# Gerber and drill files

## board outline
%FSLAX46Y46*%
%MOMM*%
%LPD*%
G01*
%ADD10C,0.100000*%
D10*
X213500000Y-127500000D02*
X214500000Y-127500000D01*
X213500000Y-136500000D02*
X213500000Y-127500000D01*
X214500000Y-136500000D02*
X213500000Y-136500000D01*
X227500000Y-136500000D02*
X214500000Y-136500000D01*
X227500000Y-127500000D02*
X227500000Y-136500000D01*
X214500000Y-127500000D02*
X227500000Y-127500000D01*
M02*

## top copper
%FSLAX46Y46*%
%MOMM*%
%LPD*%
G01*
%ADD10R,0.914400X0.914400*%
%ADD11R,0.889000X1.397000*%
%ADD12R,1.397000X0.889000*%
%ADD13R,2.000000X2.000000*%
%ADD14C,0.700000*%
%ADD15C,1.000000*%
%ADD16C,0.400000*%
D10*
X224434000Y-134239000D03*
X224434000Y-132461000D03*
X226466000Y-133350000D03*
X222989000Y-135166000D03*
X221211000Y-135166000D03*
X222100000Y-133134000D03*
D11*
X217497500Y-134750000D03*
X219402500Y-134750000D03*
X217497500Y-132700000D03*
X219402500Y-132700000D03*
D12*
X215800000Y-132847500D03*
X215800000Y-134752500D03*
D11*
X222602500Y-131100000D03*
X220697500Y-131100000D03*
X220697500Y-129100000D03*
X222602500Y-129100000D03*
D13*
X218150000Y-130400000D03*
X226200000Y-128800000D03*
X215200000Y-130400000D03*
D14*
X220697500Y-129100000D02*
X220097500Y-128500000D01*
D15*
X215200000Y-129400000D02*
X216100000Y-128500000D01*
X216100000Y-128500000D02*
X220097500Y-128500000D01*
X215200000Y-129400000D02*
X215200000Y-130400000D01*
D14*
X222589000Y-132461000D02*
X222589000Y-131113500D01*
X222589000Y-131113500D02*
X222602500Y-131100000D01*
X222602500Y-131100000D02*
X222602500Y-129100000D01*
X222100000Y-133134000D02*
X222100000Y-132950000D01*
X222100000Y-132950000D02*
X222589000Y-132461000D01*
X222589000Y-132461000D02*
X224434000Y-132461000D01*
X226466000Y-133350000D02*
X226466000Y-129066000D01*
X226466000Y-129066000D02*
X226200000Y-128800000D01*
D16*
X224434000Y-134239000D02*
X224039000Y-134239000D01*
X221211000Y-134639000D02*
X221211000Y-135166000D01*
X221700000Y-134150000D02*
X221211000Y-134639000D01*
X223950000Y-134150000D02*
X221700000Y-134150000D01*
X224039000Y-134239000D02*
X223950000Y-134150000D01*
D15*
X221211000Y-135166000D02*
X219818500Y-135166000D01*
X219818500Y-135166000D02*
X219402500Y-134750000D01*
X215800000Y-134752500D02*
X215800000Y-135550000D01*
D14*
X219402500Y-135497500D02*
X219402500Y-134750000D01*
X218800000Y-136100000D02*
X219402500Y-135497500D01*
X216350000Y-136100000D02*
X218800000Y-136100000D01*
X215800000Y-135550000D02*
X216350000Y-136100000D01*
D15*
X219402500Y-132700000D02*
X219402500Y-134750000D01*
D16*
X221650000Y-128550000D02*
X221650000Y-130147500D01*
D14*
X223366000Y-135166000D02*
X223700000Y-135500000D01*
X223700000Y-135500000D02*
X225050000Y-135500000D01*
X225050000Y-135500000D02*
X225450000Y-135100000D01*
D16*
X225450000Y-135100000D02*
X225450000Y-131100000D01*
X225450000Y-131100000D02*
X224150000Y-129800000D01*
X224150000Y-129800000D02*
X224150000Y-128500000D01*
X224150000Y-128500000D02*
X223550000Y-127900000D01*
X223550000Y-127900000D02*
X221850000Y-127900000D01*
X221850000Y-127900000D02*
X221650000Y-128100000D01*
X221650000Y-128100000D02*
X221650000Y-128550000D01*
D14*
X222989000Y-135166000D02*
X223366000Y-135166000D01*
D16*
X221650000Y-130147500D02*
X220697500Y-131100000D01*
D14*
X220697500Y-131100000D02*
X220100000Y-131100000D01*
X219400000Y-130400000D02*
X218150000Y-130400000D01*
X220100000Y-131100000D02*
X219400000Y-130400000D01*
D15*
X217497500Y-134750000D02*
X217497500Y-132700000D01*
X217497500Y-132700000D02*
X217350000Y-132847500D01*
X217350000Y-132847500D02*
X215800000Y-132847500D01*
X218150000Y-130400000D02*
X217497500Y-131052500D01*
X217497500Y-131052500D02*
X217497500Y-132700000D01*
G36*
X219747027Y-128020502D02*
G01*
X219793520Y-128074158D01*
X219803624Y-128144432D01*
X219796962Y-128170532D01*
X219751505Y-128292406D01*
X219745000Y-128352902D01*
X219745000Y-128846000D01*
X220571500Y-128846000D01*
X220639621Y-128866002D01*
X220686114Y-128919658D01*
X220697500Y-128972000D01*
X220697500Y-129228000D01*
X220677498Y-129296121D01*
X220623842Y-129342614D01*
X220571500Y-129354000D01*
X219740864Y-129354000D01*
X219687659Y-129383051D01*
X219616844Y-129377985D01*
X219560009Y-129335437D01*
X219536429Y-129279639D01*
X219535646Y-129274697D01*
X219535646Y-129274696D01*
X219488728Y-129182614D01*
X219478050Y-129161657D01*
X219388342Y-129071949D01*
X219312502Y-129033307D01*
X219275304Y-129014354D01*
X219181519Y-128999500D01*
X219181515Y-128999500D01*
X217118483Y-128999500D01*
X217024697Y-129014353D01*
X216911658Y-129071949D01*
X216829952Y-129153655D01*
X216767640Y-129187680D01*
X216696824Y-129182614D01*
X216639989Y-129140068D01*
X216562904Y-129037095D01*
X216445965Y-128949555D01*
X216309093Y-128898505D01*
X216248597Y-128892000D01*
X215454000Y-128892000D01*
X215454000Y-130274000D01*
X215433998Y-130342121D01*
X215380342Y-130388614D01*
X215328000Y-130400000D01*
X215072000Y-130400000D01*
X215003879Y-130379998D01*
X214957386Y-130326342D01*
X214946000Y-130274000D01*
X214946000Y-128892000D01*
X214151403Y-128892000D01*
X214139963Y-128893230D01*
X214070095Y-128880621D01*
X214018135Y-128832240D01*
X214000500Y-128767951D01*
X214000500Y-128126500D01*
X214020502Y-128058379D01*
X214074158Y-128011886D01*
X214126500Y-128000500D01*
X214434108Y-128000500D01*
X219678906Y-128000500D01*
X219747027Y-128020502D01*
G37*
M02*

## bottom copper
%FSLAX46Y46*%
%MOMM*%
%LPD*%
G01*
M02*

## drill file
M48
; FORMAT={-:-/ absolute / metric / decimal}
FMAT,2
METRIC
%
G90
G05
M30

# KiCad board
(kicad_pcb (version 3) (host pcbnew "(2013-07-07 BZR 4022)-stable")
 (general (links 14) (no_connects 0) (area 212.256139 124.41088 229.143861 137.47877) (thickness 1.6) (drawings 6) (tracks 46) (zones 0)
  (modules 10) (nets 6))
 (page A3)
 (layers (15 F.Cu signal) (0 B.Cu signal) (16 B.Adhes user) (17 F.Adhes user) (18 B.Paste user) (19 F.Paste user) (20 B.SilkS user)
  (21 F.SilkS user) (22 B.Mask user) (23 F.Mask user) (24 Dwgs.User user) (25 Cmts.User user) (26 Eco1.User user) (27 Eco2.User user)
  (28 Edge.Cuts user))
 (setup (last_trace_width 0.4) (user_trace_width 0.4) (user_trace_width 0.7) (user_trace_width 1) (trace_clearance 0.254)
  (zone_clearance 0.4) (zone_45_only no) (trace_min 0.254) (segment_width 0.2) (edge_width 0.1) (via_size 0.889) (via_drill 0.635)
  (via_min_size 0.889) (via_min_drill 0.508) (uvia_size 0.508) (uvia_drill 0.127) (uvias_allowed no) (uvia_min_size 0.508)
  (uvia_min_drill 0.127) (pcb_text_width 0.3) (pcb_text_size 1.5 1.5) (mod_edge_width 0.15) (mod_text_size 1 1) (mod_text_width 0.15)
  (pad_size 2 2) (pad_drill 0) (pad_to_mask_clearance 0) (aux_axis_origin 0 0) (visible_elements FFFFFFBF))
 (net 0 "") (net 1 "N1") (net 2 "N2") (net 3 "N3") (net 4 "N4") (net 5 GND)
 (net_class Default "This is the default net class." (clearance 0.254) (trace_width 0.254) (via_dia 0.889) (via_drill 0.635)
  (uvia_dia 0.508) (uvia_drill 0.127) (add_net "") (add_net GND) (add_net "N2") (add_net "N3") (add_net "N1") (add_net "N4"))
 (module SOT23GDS (layer F.Cu) (at 225.45 133.35 90)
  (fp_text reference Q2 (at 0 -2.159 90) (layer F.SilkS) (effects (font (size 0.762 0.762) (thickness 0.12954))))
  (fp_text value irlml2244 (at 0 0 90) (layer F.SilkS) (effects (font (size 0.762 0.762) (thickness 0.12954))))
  (pad S smd rect (at -0.889 -1.016 90) (size 0.9144 0.9144) (layers F.Cu F.Paste F.Mask) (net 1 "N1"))
  (pad G smd rect (at 0.889 -1.016 90) (size 0.9144 0.9144) (layers F.Cu F.Paste F.Mask) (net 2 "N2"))
  (pad D smd rect (at 0 1.016 90) (size 0.9144 0.9144) (layers F.Cu F.Paste F.Mask) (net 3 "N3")))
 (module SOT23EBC (layer F.Cu) (at 222.1 134.15 180)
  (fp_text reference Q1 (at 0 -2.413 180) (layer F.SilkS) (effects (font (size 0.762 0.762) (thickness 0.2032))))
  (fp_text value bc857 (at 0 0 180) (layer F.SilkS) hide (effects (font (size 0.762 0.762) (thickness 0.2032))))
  (pad 1 smd rect (at -0.889 -1.016 180) (size 0.9144 0.9144) (layers F.Cu F.Paste F.Mask) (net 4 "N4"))
  (pad 2 smd rect (at 0.889 -1.016 180) (size 0.9144 0.9144) (layers F.Cu F.Paste F.Mask) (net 1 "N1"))
  (pad 3 smd rect (at 0 1.016 180) (size 0.9144 0.9144) (layers F.Cu F.Paste F.Mask) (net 2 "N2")))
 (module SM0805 (layer F.Cu) (at 218.45 134.75)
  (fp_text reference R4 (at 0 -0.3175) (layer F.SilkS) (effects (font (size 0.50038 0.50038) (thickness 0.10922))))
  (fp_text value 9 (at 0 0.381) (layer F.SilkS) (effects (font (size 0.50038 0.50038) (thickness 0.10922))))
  (pad 1 smd rect (at -0.9525 0) (size 0.889 1.397) (layers F.Cu F.Paste F.Mask) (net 4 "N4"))
  (pad 2 smd rect (at 0.9525 0) (size 0.889 1.397) (layers F.Cu F.Paste F.Mask) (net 1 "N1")))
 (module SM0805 (layer F.Cu) (at 218.45 132.7)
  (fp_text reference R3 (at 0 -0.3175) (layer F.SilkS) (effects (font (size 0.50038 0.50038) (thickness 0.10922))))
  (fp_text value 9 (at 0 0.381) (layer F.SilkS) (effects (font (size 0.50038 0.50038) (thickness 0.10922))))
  (pad 1 smd rect (at -0.9525 0) (size 0.889 1.397) (layers F.Cu F.Paste F.Mask) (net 4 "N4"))
  (pad 2 smd rect (at 0.9525 0) (size 0.889 1.397) (layers F.Cu F.Paste F.Mask) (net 1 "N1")))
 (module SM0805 (layer F.Cu) (at 215.8 133.8 270)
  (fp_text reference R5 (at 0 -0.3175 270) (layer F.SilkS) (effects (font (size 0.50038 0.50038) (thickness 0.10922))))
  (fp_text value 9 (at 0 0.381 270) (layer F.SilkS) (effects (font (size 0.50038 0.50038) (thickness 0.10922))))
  (pad 1 smd rect (at -0.9525 0 270) (size 0.889 1.397) (layers F.Cu F.Paste F.Mask) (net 4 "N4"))
  (pad 2 smd rect (at 0.9525 0 270) (size 0.889 1.397) (layers F.Cu F.Paste F.Mask) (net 1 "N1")))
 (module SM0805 (layer F.Cu) (at 221.65 131.1 180)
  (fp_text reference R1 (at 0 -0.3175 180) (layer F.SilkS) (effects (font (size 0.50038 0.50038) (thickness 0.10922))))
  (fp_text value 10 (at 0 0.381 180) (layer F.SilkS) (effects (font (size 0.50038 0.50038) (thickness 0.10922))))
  (pad 1 smd rect (at -0.9525 0 180) (size 0.889 1.397) (layers F.Cu F.Paste F.Mask) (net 2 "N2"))
  (pad 2 smd rect (at 0.9525 0 180) (size 0.889 1.397) (layers F.Cu F.Paste F.Mask) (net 4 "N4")))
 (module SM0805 (layer F.Cu) (at 221.65 129.1)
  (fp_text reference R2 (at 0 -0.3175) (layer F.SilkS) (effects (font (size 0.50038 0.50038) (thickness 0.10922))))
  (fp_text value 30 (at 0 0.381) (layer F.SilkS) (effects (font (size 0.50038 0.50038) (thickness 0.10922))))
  (pad 1 smd rect (at -0.9525 0) (size 0.889 1.397) (layers F.Cu F.Paste F.Mask) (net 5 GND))
  (pad 2 smd rect (at 0.9525 0) (size 0.889 1.397) (layers F.Cu F.Paste F.Mask) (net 2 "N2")))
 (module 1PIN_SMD (layer F.Cu) (at 218.15 130.4)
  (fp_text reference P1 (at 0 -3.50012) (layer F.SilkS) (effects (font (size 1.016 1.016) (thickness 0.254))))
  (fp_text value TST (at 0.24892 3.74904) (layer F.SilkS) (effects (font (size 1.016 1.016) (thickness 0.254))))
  (pad 1 smd rect (at 0 0) (size 2 2) (layers F.Cu F.Paste F.SilkS F.Mask) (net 4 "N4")))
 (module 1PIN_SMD (layer F.Cu) (at 226.2 128.8)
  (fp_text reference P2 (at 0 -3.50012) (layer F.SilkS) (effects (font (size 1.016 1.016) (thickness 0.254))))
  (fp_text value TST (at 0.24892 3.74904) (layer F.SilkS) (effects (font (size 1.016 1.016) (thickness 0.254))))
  (pad 1 smd rect (at 0 0) (size 2 2) (layers F.Cu F.Paste F.SilkS F.Mask) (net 3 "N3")))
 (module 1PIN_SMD (layer F.Cu) (at 215.2 130.4)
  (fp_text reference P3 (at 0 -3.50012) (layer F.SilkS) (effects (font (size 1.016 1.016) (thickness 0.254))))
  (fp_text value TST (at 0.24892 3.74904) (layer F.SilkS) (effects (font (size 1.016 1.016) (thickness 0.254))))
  (pad 1 smd rect (at 0 0) (size 2 2) (layers F.Cu F.Paste F.SilkS F.Mask) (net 5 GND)))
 (gr_line (start 213.5 127.5) (end 214.5 127.5) (angle 90) (layer Edge.Cuts) (width 0.1))
 (gr_line (start 213.5 136.5) (end 213.5 127.5) (angle 90) (layer Edge.Cuts) (width 0.1))
 (gr_line (start 214.5 136.5) (end 213.5 136.5) (angle 90) (layer Edge.Cuts) (width 0.1))
 (gr_line (start 227.5 136.5) (end 214.5 136.5) (angle 90) (layer Edge.Cuts) (width 0.1))
 (gr_line (start 227.5 127.5) (end 227.5 136.5) (angle 90) (layer Edge.Cuts) (width 0.1))
 (gr_line (start 214.5 127.5) (end 227.5 127.5) (angle 90) (layer Edge.Cuts) (width 0.1))
 (segment (start 220.6975 129.1) (end 220.0975 128.5) (width 0.7) (layer F.Cu) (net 5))
 (segment (start 215.2 129.4) (end 216.1 128.5) (width 1) (layer F.Cu) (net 5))
 (segment (start 216.1 128.5) (end 220.0975 128.5) (width 1) (layer F.Cu) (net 5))
 (segment (start 215.2 129.4) (end 215.2 130.4) (width 1) (layer F.Cu) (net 5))
 (segment (start 222.589 132.461) (end 222.589 131.1135) (width 0.7) (layer F.Cu) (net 2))
 (segment (start 222.589 131.1135) (end 222.6025 131.1) (width 0.7) (layer F.Cu) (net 2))
 (segment (start 222.6025 131.1) (end 222.6025 129.1) (width 0.7) (layer F.Cu) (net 2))
 (segment (start 222.1 133.134) (end 222.1 132.95) (width 0.7) (layer F.Cu) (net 2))
 (segment (start 222.1 132.95) (end 222.589 132.461) (width 0.7) (layer F.Cu) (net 2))
 (segment (start 222.589 132.461) (end 224.434 132.461) (width 0.7) (layer F.Cu) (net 2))
 (segment (start 226.466 133.35) (end 226.466 129.066) (width 0.7) (layer F.Cu) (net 3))
 (segment (start 226.466 129.066) (end 226.2 128.8) (width 0.7) (layer F.Cu) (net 3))
 (segment (start 224.434 134.239) (end 224.039 134.239) (width 0.4) (layer F.Cu) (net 1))
 (segment (start 221.211 134.639) (end 221.211 135.166) (width 0.4) (layer F.Cu) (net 1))
 (segment (start 221.7 134.15) (end 221.211 134.639) (width 0.4) (layer F.Cu) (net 1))
 (segment (start 223.95 134.15) (end 221.7 134.15) (width 0.4) (layer F.Cu) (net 1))
 (segment (start 224.039 134.239) (end 223.95 134.15) (width 0.4) (layer F.Cu) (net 1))
 (segment (start 221.211 135.166) (end 219.8185 135.166) (width 1) (layer F.Cu) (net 1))
 (segment (start 219.8185 135.166) (end 219.4025 134.75) (width 1) (layer F.Cu) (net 1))
 (segment (start 215.8 134.7525) (end 215.8 135.55) (width 1) (layer F.Cu) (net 1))
 (segment (start 219.4025 135.4975) (end 219.4025 134.75) (width 0.7) (layer F.Cu) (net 1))
 (segment (start 218.8 136.1) (end 219.4025 135.4975) (width 0.7) (layer F.Cu) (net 1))
 (segment (start 216.35 136.1) (end 218.8 136.1) (width 0.7) (layer F.Cu) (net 1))
 (segment (start 215.8 135.55) (end 216.35 136.1) (width 0.7) (layer F.Cu) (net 1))
 (segment (start 219.4025 132.7) (end 219.4025 134.75) (width 1) (layer F.Cu) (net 1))
 (segment (start 221.65 128.55) (end 221.65 130.1475) (width 0.4) (layer F.Cu) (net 4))
 (segment (start 223.366 135.166) (end 223.7 135.5) (width 0.7) (layer F.Cu) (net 4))
 (segment (start 223.7 135.5) (end 225.05 135.5) (width 0.7) (layer F.Cu) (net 4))
 (segment (start 225.05 135.5) (end 225.45 135.1) (width 0.7) (layer F.Cu) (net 4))
 (segment (start 225.45 135.1) (end 225.45 131.1) (width 0.4) (layer F.Cu) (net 4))
 (segment (start 225.45 131.1) (end 224.15 129.8) (width 0.4) (layer F.Cu) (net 4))
 (segment (start 224.15 129.8) (end 224.15 128.5) (width 0.4) (layer F.Cu) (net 4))
 (segment (start 224.15 128.5) (end 223.55 127.9) (width 0.4) (layer F.Cu) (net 4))
 (segment (start 223.55 127.9) (end 221.85 127.9) (width 0.4) (layer F.Cu) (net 4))
 (segment (start 221.85 127.9) (end 221.65 128.1) (width 0.4) (layer F.Cu) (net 4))
 (segment (start 221.65 128.1) (end 221.65 128.55) (width 0.4) (layer F.Cu) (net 4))
 (segment (start 222.989 135.166) (end 223.366 135.166) (width 0.7) (layer F.Cu) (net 4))
 (segment (start 221.65 130.1475) (end 220.6975 131.1) (width 0.4) (layer F.Cu) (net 4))
 (segment (start 220.6975 131.1) (end 220.1 131.1) (width 0.7) (layer F.Cu) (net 4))
 (segment (start 219.4 130.4) (end 218.15 130.4) (width 0.7) (layer F.Cu) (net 4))
 (segment (start 220.1 131.1) (end 219.4 130.4) (width 0.7) (layer F.Cu) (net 4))
 (segment (start 217.4975 134.75) (end 217.4975 132.7) (width 1) (layer F.Cu) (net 4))
 (segment (start 217.4975 132.7) (end 217.35 132.8475) (width 1) (layer F.Cu) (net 4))
 (segment (start 217.35 132.8475) (end 215.8 132.8475) (width 1) (layer F.Cu) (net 4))
 (segment (start 218.15 130.4) (end 217.4975 131.0525) (width 1) (layer F.Cu) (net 4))
 (segment (start 217.4975 131.0525) (end 217.4975 132.7) (width 1) (layer F.Cu) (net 4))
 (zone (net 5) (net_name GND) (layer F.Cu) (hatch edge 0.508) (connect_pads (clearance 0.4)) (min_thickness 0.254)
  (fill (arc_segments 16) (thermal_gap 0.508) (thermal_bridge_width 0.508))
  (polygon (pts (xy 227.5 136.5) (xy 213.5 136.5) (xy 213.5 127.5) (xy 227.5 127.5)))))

